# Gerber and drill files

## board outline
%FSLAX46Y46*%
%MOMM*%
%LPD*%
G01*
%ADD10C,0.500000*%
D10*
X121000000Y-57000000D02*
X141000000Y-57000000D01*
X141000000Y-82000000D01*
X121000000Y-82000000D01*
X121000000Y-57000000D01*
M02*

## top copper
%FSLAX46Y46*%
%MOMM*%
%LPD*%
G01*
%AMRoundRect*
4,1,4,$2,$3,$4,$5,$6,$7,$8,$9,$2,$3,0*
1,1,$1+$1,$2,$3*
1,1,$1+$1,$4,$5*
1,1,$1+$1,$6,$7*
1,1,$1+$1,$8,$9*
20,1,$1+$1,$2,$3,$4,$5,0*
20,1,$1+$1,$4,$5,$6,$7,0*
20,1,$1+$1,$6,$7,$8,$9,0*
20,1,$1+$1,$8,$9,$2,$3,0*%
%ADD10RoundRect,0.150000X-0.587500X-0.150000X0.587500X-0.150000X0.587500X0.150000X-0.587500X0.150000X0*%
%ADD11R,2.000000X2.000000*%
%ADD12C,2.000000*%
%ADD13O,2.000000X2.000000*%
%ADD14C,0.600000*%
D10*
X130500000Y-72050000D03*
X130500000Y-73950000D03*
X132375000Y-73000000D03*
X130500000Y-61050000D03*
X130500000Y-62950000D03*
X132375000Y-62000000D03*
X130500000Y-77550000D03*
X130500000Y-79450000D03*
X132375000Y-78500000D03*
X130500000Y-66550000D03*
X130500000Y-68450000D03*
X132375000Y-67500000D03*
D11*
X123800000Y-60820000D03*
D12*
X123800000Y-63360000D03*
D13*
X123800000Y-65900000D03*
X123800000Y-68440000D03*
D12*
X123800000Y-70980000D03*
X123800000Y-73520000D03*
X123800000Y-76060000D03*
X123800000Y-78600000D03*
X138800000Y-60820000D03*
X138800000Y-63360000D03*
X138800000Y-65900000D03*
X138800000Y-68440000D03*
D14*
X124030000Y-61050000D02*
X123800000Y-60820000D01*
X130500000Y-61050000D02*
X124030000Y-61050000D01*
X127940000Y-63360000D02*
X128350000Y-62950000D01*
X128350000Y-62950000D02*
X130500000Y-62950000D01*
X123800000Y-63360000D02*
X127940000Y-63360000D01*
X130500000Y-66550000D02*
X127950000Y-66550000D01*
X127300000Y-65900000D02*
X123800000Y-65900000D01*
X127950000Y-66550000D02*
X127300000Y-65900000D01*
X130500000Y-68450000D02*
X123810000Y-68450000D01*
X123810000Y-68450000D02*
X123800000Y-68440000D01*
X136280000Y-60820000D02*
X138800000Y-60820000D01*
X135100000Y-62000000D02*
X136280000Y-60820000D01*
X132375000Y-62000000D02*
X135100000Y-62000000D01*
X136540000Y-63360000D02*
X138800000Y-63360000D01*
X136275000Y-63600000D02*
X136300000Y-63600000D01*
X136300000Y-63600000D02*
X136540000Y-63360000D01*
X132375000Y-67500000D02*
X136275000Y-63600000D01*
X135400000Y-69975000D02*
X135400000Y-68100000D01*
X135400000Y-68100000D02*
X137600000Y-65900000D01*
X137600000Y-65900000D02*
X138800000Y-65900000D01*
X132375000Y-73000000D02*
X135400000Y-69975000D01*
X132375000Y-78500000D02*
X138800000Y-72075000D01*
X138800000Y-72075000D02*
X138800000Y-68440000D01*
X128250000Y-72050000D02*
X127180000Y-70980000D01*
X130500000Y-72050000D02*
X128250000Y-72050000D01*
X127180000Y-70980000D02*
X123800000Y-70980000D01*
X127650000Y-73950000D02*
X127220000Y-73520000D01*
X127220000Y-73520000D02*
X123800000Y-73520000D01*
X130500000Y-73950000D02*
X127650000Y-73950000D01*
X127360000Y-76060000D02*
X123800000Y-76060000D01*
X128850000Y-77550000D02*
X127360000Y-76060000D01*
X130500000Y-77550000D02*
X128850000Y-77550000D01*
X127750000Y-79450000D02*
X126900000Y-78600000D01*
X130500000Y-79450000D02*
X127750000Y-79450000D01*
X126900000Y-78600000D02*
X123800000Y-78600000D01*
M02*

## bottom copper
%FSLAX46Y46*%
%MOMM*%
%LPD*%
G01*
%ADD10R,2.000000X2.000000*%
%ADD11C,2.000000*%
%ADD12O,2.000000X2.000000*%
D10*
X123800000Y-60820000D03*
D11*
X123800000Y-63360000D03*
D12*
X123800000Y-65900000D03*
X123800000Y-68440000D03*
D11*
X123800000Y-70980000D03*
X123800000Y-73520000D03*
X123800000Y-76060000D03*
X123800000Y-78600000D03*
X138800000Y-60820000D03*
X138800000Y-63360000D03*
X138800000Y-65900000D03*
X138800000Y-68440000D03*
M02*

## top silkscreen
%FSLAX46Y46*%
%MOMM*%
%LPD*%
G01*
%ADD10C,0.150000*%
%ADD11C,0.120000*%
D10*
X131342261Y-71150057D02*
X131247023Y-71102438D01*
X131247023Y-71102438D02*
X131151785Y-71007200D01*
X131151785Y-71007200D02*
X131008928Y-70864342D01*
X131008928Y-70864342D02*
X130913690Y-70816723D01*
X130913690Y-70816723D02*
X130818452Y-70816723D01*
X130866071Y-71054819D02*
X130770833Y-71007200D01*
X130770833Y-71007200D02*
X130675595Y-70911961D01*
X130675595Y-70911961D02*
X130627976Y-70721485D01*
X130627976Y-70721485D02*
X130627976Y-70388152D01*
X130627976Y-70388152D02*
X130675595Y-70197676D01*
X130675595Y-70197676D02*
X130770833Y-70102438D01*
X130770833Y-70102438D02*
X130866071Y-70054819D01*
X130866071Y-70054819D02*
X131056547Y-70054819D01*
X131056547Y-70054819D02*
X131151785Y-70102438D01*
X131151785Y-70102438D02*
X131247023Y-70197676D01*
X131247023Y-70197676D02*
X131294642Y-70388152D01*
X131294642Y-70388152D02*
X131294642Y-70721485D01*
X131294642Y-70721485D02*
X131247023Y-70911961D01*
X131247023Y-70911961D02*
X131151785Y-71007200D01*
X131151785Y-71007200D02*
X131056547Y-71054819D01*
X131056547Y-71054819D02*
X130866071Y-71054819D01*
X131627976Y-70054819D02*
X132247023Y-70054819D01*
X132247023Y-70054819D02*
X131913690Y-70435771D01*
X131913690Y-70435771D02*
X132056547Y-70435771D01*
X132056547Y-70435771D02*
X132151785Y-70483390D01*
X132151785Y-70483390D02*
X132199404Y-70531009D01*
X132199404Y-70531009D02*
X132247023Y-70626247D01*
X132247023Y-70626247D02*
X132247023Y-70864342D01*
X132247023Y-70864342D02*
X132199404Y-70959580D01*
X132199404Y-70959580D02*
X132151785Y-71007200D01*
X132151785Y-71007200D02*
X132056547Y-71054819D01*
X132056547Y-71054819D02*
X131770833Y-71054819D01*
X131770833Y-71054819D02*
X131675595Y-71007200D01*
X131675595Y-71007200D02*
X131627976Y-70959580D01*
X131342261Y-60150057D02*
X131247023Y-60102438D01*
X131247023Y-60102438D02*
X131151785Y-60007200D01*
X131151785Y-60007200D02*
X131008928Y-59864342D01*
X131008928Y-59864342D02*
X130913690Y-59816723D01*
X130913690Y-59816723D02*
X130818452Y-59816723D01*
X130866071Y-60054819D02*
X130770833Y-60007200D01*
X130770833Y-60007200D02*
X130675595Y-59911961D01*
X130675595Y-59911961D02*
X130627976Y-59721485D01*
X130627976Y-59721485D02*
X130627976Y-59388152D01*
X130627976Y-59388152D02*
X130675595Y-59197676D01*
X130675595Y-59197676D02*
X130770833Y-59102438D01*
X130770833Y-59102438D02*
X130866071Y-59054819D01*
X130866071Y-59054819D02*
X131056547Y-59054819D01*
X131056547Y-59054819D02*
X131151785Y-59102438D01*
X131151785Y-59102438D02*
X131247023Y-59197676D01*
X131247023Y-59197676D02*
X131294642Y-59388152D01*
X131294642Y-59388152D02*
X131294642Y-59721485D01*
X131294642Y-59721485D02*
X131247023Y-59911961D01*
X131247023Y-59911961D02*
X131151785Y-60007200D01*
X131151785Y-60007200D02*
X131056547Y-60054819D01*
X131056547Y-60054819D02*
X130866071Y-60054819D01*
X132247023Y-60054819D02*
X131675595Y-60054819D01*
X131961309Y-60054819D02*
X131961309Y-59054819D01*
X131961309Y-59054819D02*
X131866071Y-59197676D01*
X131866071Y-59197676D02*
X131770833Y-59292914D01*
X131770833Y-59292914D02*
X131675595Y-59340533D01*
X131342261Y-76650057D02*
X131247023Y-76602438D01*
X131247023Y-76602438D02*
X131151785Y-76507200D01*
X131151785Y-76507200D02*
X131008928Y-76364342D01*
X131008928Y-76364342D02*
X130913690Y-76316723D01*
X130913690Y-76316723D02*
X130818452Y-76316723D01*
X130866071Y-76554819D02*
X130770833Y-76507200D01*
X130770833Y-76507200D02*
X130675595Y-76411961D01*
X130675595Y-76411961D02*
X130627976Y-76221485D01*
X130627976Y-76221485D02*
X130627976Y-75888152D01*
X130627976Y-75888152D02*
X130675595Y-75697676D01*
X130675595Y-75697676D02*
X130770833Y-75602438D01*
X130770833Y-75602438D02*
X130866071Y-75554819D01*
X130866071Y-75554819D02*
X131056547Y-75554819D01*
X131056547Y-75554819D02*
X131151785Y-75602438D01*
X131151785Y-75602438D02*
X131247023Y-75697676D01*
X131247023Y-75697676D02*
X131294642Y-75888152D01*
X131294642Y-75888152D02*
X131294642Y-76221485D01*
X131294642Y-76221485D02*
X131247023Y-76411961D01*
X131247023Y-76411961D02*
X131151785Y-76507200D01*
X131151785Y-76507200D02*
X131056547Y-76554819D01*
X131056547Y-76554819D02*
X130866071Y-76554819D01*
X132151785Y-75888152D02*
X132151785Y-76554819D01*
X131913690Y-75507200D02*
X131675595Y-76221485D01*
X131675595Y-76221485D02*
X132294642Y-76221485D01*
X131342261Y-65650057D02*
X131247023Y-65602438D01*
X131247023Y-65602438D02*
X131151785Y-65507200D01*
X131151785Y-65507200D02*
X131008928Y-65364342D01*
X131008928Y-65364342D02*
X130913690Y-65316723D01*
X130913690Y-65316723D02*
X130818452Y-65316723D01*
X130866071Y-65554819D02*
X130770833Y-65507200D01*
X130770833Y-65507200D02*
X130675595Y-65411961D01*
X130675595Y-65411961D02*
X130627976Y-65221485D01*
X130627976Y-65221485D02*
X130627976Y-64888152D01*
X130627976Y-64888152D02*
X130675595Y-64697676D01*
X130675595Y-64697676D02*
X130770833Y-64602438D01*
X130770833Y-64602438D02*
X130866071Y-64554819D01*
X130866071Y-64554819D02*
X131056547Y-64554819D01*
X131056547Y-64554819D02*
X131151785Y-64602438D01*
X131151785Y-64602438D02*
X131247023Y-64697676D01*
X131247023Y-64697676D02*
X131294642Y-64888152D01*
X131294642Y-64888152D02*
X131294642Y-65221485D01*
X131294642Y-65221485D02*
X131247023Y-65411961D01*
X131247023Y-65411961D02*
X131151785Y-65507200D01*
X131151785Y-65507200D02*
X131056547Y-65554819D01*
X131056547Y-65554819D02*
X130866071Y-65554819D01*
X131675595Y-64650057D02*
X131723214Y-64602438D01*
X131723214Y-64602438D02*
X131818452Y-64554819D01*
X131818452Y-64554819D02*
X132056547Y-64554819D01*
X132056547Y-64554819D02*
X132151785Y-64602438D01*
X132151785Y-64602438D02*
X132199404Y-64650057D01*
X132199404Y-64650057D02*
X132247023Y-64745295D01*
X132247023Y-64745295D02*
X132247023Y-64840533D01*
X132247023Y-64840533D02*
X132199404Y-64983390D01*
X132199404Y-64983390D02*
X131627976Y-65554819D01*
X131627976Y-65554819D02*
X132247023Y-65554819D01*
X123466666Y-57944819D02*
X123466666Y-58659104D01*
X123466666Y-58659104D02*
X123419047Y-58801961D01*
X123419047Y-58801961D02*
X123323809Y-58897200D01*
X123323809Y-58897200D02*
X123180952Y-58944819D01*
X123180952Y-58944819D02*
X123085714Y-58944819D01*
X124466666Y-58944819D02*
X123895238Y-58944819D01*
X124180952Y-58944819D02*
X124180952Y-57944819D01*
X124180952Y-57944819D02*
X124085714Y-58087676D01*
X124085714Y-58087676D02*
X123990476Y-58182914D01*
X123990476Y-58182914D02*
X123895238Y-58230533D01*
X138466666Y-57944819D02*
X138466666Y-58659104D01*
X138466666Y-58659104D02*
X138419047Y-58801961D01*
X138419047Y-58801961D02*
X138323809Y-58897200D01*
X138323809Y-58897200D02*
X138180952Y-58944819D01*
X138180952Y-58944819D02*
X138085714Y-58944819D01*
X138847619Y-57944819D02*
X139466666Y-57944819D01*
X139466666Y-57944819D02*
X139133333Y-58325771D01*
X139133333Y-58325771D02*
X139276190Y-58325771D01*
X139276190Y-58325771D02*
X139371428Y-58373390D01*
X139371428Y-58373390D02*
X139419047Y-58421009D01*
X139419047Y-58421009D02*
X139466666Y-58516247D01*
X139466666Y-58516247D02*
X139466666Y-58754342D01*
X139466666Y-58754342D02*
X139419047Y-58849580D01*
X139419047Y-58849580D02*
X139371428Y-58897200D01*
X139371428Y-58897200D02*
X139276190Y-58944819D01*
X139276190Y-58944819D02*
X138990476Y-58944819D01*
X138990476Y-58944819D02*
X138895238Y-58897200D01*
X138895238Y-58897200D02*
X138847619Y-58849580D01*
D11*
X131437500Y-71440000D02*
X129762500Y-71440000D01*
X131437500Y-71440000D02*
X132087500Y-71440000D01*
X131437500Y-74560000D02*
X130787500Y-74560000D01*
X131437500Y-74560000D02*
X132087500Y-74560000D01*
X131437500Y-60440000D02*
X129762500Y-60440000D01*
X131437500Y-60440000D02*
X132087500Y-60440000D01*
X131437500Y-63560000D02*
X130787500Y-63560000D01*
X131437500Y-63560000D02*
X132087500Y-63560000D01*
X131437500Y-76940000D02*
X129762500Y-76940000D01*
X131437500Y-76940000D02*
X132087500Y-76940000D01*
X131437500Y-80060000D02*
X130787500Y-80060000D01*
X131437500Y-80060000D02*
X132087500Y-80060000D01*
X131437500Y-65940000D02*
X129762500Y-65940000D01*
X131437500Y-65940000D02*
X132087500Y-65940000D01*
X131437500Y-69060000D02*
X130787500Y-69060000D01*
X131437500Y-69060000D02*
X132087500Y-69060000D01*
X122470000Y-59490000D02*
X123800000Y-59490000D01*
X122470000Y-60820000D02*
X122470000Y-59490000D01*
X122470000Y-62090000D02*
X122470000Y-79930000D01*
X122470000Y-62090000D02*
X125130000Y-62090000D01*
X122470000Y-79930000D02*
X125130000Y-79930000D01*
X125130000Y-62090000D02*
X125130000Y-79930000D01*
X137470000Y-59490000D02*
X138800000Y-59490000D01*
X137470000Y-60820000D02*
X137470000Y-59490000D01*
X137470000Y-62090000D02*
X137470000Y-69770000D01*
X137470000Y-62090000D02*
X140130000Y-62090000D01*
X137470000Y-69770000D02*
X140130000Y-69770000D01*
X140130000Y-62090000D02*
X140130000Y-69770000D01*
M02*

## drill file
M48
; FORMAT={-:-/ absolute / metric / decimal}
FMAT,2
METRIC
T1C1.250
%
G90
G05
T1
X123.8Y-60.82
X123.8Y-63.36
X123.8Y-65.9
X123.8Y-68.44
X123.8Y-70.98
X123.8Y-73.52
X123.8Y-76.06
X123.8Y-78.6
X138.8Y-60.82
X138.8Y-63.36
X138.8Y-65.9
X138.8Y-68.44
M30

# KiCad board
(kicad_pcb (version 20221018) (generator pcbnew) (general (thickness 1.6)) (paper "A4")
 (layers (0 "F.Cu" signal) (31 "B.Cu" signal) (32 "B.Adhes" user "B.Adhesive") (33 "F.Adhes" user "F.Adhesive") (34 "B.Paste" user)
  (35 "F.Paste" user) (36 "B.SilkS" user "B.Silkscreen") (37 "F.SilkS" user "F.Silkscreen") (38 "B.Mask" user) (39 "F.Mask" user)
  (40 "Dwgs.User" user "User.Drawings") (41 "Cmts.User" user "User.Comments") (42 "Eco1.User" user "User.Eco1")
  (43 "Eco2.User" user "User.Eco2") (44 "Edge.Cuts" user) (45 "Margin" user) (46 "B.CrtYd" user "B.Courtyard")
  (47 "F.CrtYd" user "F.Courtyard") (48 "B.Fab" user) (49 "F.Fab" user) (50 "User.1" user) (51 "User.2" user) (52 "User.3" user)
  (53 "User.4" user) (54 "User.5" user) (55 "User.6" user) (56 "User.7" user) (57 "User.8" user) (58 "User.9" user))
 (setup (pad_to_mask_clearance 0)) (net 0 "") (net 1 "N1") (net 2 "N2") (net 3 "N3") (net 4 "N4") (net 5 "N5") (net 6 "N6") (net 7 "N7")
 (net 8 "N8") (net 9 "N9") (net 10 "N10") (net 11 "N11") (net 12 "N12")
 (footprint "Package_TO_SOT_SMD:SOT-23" (layer "F.Cu") (at 131.4375 73)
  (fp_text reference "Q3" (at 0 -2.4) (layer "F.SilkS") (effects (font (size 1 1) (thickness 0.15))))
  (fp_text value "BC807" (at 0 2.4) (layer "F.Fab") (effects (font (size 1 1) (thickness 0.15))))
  (fp_line (start 0 -1.56) (end -1.675 -1.56) (stroke (width 0.12) (type solid)) (layer "F.SilkS"))
  (fp_line (start 0 -1.56) (end 0.65 -1.56) (stroke (width 0.12) (type solid)) (layer "F.SilkS"))
  (fp_line (start 0 1.56) (end -0.65 1.56) (stroke (width 0.12) (type solid)) (layer "F.SilkS"))
  (fp_line (start 0 1.56) (end 0.65 1.56) (stroke (width 0.12) (type solid)) (layer "F.SilkS"))
  (pad "1" smd roundrect (at -0.9375 -0.95) (size 1.475 0.6) (layers "F.Cu" "F.Paste" "F.Mask") (roundrect_rratio 0.25) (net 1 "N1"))
  (pad "2" smd roundrect (at -0.9375 0.95) (size 1.475 0.6) (layers "F.Cu" "F.Paste" "F.Mask") (roundrect_rratio 0.25) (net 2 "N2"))
  (pad "3" smd roundrect (at 0.9375 0) (size 1.475 0.6) (layers "F.Cu" "F.Paste" "F.Mask") (roundrect_rratio 0.25) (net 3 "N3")))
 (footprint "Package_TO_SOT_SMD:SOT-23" (layer "F.Cu") (at 131.4375 62)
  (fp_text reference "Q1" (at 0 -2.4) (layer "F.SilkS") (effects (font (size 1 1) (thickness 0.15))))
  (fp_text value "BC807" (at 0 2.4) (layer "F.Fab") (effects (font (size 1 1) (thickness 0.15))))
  (fp_line (start 0 -1.56) (end -1.675 -1.56) (stroke (width 0.12) (type solid)) (layer "F.SilkS"))
  (fp_line (start 0 -1.56) (end 0.65 -1.56) (stroke (width 0.12) (type solid)) (layer "F.SilkS"))
  (fp_line (start 0 1.56) (end -0.65 1.56) (stroke (width 0.12) (type solid)) (layer "F.SilkS"))
  (fp_line (start 0 1.56) (end 0.65 1.56) (stroke (width 0.12) (type solid)) (layer "F.SilkS"))
  (pad "1" smd roundrect (at -0.9375 -0.95) (size 1.475 0.6) (layers "F.Cu" "F.Paste" "F.Mask") (roundrect_rratio 0.25) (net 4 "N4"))
  (pad "2" smd roundrect (at -0.9375 0.95) (size 1.475 0.6) (layers "F.Cu" "F.Paste" "F.Mask") (roundrect_rratio 0.25) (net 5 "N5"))
  (pad "3" smd roundrect (at 0.9375 0) (size 1.475 0.6) (layers "F.Cu" "F.Paste" "F.Mask") (roundrect_rratio 0.25) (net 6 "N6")))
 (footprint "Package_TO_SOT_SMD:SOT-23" (layer "F.Cu") (at 131.4375 78.5)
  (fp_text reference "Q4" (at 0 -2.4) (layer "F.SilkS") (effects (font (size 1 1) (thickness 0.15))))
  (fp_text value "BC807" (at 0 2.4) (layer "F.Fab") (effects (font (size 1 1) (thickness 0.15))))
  (fp_line (start 0 -1.56) (end -1.675 -1.56) (stroke (width 0.12) (type solid)) (layer "F.SilkS"))
  (fp_line (start 0 -1.56) (end 0.65 -1.56) (stroke (width 0.12) (type solid)) (layer "F.SilkS"))
  (fp_line (start 0 1.56) (end -0.65 1.56) (stroke (width 0.12) (type solid)) (layer "F.SilkS"))
  (fp_line (start 0 1.56) (end 0.65 1.56) (stroke (width 0.12) (type solid)) (layer "F.SilkS"))
  (pad "1" smd roundrect (at -0.9375 -0.95) (size 1.475 0.6) (layers "F.Cu" "F.Paste" "F.Mask") (roundrect_rratio 0.25) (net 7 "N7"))
  (pad "2" smd roundrect (at -0.9375 0.95) (size 1.475 0.6) (layers "F.Cu" "F.Paste" "F.Mask") (roundrect_rratio 0.25) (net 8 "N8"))
  (pad "3" smd roundrect (at 0.9375 0) (size 1.475 0.6) (layers "F.Cu" "F.Paste" "F.Mask") (roundrect_rratio 0.25) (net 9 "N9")))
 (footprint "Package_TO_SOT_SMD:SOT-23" (layer "F.Cu") (at 131.4375 67.5)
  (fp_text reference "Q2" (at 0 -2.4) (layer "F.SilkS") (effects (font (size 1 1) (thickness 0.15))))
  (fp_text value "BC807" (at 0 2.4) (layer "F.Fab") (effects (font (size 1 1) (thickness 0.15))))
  (fp_line (start 0 -1.56) (end -1.675 -1.56) (stroke (width 0.12) (type solid)) (layer "F.SilkS"))
  (fp_line (start 0 -1.56) (end 0.65 -1.56) (stroke (width 0.12) (type solid)) (layer "F.SilkS"))
  (fp_line (start 0 1.56) (end -0.65 1.56) (stroke (width 0.12) (type solid)) (layer "F.SilkS"))
  (fp_line (start 0 1.56) (end 0.65 1.56) (stroke (width 0.12) (type solid)) (layer "F.SilkS"))
  (pad "1" smd roundrect (at -0.9375 -0.95) (size 1.475 0.6) (layers "F.Cu" "F.Paste" "F.Mask") (roundrect_rratio 0.25) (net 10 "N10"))
  (pad "2" smd roundrect (at -0.9375 0.95) (size 1.475 0.6) (layers "F.Cu" "F.Paste" "F.Mask") (roundrect_rratio 0.25) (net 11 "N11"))
  (pad "3" smd roundrect (at 0.9375 0) (size 1.475 0.6) (layers "F.Cu" "F.Paste" "F.Mask") (roundrect_rratio 0.25) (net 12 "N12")))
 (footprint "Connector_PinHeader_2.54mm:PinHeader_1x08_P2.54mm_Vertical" (layer "F.Cu") (at 123.8 60.82)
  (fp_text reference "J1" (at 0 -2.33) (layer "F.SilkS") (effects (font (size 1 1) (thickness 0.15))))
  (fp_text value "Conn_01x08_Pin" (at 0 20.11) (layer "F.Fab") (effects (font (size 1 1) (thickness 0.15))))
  (fp_line (start -1.33 -1.33) (end 0 -1.33) (stroke (width 0.12) (type solid)) (layer "F.SilkS"))
  (fp_line (start -1.33 0) (end -1.33 -1.33) (stroke (width 0.12) (type solid)) (layer "F.SilkS"))
  (fp_line (start -1.33 1.27) (end -1.33 19.11) (stroke (width 0.12) (type solid)) (layer "F.SilkS"))
  (fp_line (start -1.33 1.27) (end 1.33 1.27) (stroke (width 0.12) (type solid)) (layer "F.SilkS"))
  (fp_line (start -1.33 19.11) (end 1.33 19.11) (stroke (width 0.12) (type solid)) (layer "F.SilkS"))
  (fp_line (start 1.33 1.27) (end 1.33 19.11) (stroke (width 0.12) (type solid)) (layer "F.SilkS"))
  (pad "1" thru_hole rect (at 0 0) (size 2 2) (drill 1.25) (layers "*.Cu" "*.Mask") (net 4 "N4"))
  (pad "2" thru_hole circle (at 0 2.54) (size 2 2) (drill 1.25) (layers "*.Cu" "*.Mask") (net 5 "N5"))
  (pad "3" thru_hole oval (at 0 5.08) (size 2 2) (drill 1.25) (layers "*.Cu" "*.Mask") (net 10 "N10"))
  (pad "4" thru_hole oval (at 0 7.62) (size 2 2) (drill 1.25) (layers "*.Cu" "*.Mask") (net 11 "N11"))
  (pad "5" thru_hole circle (at 0 10.16) (size 2 2) (drill 1.25) (layers "*.Cu" "*.Mask") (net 1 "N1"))
  (pad "6" thru_hole circle (at 0 12.7) (size 2 2) (drill 1.25) (layers "*.Cu" "*.Mask") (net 2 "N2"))
  (pad "7" thru_hole circle (at 0 15.24) (size 2 2) (drill 1.25) (layers "*.Cu" "*.Mask") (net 7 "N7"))
  (pad "8" thru_hole circle (at 0 17.78) (size 2 2) (drill 1.25) (layers "*.Cu" "*.Mask") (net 8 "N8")))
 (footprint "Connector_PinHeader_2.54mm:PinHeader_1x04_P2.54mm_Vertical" (layer "F.Cu") (at 138.8 60.82)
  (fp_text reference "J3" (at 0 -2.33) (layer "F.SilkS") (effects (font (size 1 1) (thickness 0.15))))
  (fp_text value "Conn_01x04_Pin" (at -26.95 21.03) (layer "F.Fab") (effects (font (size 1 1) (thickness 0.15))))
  (fp_line (start -1.33 -1.33) (end 0 -1.33) (stroke (width 0.12) (type solid)) (layer "F.SilkS"))
  (fp_line (start -1.33 0) (end -1.33 -1.33) (stroke (width 0.12) (type solid)) (layer "F.SilkS"))
  (fp_line (start -1.33 1.27) (end -1.33 8.95) (stroke (width 0.12) (type solid)) (layer "F.SilkS"))
  (fp_line (start -1.33 1.27) (end 1.33 1.27) (stroke (width 0.12) (type solid)) (layer "F.SilkS"))
  (fp_line (start -1.33 8.95) (end 1.33 8.95) (stroke (width 0.12) (type solid)) (layer "F.SilkS"))
  (fp_line (start 1.33 1.27) (end 1.33 8.95) (stroke (width 0.12) (type solid)) (layer "F.SilkS"))
  (pad "1" thru_hole circle (at 0 0) (size 2 2) (drill 1.25) (layers "*.Cu" "*.Mask") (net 6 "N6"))
  (pad "2" thru_hole circle (at 0 2.54) (size 2 2) (drill 1.25) (layers "*.Cu" "*.Mask") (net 12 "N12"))
  (pad "3" thru_hole circle (at 0 5.08) (size 2 2) (drill 1.25) (layers "*.Cu" "*.Mask") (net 3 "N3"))
  (pad "4" thru_hole circle (at 0 7.62) (size 2 2) (drill 1.25) (layers "*.Cu" "*.Mask") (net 9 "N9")))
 (gr_rect (start 121 57) (end 141 82) (stroke (width 0.5) (type default)) (fill none) (layer "Edge.Cuts"))
 (segment (start 124.03 61.05) (end 123.8 60.82) (width 0.6) (layer "F.Cu") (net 4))
 (segment (start 130.5 61.05) (end 124.03 61.05) (width 0.6) (layer "F.Cu") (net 4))
 (segment (start 127.94 63.36) (end 128.35 62.95) (width 0.6) (layer "F.Cu") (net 5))
 (segment (start 128.35 62.95) (end 130.5 62.95) (width 0.6) (layer "F.Cu") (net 5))
 (segment (start 123.8 63.36) (end 127.94 63.36) (width 0.6) (layer "F.Cu") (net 5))
 (segment (start 130.5 66.55) (end 127.95 66.55) (width 0.6) (layer "F.Cu") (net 10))
 (segment (start 127.3 65.9) (end 123.8 65.9) (width 0.6) (layer "F.Cu") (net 10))
 (segment (start 127.95 66.55) (end 127.3 65.9) (width 0.6) (layer "F.Cu") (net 10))
 (segment (start 130.5 68.45) (end 123.81 68.45) (width 0.6) (layer "F.Cu") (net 11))
 (segment (start 123.81 68.45) (end 123.8 68.44) (width 0.6) (layer "F.Cu") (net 11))
 (segment (start 136.28 60.82) (end 138.8 60.82) (width 0.6) (layer "F.Cu") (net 6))
 (segment (start 135.1 62) (end 136.28 60.82) (width 0.6) (layer "F.Cu") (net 6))
 (segment (start 132.375 62) (end 135.1 62) (width 0.6) (layer "F.Cu") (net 6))
 (segment (start 136.54 63.36) (end 138.8 63.36) (width 0.6) (layer "F.Cu") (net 12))
 (segment (start 136.275 63.6) (end 136.3 63.6) (width 0.6) (layer "F.Cu") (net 12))
 (segment (start 136.3 63.6) (end 136.54 63.36) (width 0.6) (layer "F.Cu") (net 12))
 (segment (start 132.375 67.5) (end 136.275 63.6) (width 0.6) (layer "F.Cu") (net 12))
 (segment (start 135.4 69.975) (end 135.4 68.1) (width 0.6) (layer "F.Cu") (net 3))
 (segment (start 135.4 68.1) (end 137.6 65.9) (width 0.6) (layer "F.Cu") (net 3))
 (segment (start 137.6 65.9) (end 138.8 65.9) (width 0.6) (layer "F.Cu") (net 3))
 (segment (start 132.375 73) (end 135.4 69.975) (width 0.6) (layer "F.Cu") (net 3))
 (segment (start 132.375 78.5) (end 138.8 72.075) (width 0.6) (layer "F.Cu") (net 9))
 (segment (start 138.8 72.075) (end 138.8 68.44) (width 0.6) (layer "F.Cu") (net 9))
 (segment (start 128.25 72.05) (end 127.18 70.98) (width 0.6) (layer "F.Cu") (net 1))
 (segment (start 130.5 72.05) (end 128.25 72.05) (width 0.6) (layer "F.Cu") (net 1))
 (segment (start 127.18 70.98) (end 123.8 70.98) (width 0.6) (layer "F.Cu") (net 1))
 (segment (start 127.65 73.95) (end 127.22 73.52) (width 0.6) (layer "F.Cu") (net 2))
 (segment (start 127.22 73.52) (end 123.8 73.52) (width 0.6) (layer "F.Cu") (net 2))
 (segment (start 130.5 73.95) (end 127.65 73.95) (width 0.6) (layer "F.Cu") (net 2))
 (segment (start 127.36 76.06) (end 123.8 76.06) (width 0.6) (layer "F.Cu") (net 7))
 (segment (start 128.85 77.55) (end 127.36 76.06) (width 0.6) (layer "F.Cu") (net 7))
 (segment (start 130.5 77.55) (end 128.85 77.55) (width 0.6) (layer "F.Cu") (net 7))
 (segment (start 127.75 79.45) (end 126.9 78.6) (width 0.6) (layer "F.Cu") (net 8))
 (segment (start 130.5 79.45) (end 127.75 79.45) (width 0.6) (layer "F.Cu") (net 8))
 (segment (start 126.9 78.6) (end 123.8 78.6) (width 0.6) (layer "F.Cu") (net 8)))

